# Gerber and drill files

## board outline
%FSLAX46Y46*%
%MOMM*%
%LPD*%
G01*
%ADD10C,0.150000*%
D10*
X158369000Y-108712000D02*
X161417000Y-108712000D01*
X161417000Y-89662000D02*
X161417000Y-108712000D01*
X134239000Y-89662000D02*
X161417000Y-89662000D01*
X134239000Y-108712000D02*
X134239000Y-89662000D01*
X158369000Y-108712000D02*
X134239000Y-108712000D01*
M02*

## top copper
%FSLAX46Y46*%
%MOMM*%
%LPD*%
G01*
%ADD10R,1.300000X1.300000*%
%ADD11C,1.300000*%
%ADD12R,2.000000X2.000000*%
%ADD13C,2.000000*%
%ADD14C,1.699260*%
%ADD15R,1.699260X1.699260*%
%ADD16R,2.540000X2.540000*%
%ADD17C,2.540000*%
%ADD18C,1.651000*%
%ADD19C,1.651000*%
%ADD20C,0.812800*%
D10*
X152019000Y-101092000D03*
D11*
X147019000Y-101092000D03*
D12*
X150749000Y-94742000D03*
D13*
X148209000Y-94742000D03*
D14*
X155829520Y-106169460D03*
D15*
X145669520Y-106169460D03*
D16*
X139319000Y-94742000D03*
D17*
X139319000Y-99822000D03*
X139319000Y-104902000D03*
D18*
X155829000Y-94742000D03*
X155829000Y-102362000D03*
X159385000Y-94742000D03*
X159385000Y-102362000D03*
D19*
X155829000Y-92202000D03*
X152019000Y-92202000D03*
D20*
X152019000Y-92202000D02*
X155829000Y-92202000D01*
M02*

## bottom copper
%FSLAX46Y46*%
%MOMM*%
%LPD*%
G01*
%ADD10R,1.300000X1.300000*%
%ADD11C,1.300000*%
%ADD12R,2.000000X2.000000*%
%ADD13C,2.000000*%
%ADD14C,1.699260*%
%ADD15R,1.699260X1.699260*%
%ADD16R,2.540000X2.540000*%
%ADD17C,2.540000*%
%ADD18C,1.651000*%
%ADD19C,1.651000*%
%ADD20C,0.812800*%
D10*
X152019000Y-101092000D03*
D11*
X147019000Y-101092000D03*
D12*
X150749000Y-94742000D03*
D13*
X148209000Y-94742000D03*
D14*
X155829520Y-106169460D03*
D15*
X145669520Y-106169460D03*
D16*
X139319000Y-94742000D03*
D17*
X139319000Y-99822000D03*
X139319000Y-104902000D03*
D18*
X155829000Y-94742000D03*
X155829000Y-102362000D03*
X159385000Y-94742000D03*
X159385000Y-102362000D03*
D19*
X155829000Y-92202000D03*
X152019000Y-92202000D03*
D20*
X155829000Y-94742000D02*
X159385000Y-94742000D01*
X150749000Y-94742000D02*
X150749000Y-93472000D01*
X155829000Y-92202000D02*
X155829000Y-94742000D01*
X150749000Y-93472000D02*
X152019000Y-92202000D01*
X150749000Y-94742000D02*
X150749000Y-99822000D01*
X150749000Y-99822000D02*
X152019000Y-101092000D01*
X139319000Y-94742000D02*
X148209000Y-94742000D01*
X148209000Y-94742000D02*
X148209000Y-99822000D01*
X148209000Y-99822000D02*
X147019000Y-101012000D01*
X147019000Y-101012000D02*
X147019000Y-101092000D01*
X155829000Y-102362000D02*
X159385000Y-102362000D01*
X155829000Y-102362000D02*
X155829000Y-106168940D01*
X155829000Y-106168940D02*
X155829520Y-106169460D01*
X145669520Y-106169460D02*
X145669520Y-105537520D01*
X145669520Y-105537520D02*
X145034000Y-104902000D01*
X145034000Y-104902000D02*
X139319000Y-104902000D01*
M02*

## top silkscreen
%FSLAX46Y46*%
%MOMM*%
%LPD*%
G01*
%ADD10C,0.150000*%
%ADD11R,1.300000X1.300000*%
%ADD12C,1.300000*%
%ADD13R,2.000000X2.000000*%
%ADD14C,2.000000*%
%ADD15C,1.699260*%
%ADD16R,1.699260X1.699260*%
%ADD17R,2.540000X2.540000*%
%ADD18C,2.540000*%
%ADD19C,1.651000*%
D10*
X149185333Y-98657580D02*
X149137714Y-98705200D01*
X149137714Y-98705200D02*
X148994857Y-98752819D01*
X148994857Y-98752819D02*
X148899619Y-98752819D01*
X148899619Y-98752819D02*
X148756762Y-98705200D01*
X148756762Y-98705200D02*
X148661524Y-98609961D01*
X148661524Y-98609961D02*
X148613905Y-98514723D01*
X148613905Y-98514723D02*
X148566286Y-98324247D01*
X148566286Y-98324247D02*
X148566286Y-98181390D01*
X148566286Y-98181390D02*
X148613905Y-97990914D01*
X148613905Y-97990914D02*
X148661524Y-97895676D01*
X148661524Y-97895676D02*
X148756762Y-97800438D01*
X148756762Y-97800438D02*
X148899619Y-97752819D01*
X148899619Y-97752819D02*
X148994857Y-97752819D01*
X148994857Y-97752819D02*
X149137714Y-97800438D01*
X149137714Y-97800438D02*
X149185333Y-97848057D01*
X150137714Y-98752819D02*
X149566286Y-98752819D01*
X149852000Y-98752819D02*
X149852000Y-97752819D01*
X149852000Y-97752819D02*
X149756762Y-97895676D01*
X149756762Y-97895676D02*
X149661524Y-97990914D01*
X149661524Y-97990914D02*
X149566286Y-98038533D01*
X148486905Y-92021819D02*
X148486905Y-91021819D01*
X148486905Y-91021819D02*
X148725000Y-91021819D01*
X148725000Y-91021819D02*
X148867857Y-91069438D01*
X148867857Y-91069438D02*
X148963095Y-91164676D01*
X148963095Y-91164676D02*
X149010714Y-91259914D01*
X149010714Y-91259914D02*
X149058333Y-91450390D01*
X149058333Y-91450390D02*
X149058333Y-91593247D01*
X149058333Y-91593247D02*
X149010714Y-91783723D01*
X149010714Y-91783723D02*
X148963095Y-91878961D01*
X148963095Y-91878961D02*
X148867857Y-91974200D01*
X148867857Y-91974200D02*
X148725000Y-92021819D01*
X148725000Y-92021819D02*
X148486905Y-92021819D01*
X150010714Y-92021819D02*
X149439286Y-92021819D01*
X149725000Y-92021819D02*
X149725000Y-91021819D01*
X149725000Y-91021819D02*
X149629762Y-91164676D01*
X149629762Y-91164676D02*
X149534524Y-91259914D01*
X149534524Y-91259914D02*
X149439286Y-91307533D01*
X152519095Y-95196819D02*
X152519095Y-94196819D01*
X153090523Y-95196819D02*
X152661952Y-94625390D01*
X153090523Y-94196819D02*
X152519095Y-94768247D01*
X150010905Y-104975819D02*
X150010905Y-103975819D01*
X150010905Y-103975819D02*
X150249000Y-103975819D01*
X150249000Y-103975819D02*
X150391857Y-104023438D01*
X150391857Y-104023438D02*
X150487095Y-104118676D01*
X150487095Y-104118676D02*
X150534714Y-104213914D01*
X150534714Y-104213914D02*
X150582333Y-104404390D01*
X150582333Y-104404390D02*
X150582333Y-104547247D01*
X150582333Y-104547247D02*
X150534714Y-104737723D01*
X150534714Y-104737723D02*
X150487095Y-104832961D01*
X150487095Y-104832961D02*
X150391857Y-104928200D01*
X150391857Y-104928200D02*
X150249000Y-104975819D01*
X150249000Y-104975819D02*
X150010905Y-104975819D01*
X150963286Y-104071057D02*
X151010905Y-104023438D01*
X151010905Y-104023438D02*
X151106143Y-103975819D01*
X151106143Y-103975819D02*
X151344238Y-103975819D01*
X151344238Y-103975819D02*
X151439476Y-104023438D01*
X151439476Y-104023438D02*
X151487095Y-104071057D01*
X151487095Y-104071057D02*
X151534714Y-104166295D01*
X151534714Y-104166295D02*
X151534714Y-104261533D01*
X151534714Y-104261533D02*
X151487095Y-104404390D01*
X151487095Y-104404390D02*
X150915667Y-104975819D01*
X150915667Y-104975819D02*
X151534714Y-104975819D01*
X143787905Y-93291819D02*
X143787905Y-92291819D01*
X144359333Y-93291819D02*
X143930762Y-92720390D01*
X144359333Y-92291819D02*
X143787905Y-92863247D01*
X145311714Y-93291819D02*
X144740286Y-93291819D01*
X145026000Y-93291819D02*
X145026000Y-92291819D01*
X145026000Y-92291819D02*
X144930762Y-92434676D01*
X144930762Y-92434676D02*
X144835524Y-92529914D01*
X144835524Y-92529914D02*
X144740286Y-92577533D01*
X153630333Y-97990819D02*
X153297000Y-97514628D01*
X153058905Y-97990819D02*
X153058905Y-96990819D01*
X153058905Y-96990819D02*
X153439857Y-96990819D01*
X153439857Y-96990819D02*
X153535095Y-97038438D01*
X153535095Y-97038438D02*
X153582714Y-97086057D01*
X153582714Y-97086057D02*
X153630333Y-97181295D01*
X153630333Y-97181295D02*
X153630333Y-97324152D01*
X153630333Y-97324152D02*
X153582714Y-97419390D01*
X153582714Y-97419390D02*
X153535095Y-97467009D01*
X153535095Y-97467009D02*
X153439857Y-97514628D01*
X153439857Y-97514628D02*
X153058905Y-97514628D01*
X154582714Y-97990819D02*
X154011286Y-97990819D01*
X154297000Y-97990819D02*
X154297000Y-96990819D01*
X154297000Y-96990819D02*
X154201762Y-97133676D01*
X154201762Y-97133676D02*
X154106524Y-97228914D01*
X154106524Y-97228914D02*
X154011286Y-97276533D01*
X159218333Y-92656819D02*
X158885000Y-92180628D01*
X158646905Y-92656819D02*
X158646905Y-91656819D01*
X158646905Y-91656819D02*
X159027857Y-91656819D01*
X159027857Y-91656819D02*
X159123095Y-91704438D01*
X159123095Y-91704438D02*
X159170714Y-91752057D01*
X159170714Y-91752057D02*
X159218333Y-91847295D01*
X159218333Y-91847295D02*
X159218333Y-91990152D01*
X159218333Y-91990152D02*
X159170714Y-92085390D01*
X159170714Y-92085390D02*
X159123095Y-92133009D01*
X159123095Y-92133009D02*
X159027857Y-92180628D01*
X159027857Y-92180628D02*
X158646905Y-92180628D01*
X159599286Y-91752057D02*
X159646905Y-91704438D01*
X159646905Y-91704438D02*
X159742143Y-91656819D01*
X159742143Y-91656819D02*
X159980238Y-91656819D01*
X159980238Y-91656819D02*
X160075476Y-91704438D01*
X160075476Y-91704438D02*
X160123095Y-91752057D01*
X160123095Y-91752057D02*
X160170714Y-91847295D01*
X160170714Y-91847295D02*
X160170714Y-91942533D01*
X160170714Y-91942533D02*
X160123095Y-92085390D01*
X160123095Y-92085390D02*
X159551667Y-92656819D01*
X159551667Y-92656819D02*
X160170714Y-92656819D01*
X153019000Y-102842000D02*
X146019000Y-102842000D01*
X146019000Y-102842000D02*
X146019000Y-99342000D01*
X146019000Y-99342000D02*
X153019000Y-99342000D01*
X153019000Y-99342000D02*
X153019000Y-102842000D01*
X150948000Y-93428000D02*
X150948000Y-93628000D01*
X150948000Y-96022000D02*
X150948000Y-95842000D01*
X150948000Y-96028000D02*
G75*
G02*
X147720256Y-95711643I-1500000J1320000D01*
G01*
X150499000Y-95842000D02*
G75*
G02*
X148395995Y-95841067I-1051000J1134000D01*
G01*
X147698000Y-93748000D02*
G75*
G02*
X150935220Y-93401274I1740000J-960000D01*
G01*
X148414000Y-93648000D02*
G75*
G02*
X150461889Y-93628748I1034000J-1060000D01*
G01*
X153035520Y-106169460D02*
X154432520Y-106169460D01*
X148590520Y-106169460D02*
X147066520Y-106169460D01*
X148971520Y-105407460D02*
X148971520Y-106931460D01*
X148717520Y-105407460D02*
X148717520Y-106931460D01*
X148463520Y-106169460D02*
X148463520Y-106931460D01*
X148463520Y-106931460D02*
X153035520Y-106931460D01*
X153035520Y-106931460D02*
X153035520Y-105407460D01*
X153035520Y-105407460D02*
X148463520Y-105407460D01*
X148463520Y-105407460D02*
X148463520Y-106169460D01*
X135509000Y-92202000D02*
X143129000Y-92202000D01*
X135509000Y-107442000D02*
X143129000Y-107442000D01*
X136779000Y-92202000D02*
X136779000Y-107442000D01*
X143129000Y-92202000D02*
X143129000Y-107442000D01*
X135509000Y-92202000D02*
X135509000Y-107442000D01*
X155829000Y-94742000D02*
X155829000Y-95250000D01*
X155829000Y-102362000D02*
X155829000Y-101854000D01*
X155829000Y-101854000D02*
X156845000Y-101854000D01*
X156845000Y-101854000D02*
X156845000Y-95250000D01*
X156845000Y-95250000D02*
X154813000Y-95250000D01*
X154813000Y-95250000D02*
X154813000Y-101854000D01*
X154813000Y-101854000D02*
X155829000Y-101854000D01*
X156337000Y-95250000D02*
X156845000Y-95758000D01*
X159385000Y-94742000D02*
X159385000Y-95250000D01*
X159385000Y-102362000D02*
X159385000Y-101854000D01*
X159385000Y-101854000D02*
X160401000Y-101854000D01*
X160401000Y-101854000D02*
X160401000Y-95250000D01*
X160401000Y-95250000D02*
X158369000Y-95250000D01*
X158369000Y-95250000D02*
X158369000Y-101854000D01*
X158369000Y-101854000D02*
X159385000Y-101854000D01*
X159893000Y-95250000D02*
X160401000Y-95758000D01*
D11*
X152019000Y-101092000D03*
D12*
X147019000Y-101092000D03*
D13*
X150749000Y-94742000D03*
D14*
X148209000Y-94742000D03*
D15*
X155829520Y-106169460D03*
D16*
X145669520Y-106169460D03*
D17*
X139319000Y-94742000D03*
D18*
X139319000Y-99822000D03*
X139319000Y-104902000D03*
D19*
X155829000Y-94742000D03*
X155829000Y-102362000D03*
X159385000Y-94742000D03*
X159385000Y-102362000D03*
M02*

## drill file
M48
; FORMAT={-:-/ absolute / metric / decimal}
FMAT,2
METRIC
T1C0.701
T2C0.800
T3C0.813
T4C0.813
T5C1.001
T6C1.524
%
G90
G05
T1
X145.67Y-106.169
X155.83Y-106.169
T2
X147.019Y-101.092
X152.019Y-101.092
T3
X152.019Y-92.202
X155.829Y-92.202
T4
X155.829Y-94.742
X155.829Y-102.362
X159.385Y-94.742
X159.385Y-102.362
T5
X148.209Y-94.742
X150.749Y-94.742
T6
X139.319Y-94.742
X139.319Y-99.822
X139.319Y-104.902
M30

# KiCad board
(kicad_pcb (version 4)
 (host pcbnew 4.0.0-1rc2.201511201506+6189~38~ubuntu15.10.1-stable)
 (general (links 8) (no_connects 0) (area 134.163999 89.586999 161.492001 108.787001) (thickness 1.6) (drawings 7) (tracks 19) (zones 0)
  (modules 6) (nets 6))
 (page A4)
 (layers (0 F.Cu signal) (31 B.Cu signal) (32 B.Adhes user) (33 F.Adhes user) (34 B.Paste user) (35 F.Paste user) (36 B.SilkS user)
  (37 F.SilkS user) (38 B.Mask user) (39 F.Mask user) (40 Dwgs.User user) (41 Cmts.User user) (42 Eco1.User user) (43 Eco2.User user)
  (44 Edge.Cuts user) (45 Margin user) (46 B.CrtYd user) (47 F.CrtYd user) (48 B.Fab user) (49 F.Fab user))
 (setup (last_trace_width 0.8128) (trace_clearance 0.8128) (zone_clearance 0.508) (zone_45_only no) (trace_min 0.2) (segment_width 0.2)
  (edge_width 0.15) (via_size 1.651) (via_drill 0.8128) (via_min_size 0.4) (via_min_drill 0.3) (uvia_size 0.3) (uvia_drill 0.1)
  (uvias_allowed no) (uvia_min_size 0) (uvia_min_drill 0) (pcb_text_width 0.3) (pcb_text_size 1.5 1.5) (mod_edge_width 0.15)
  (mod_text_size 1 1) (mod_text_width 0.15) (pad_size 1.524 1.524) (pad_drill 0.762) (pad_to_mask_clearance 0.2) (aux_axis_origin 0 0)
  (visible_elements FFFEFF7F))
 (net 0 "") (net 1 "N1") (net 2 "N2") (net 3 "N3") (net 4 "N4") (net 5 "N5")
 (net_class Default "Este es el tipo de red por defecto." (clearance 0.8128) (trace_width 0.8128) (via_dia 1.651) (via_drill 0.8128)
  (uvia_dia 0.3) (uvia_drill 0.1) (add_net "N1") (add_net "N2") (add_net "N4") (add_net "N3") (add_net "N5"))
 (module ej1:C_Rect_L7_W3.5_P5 (layer F.Cu) (at 152.019 101.092 180)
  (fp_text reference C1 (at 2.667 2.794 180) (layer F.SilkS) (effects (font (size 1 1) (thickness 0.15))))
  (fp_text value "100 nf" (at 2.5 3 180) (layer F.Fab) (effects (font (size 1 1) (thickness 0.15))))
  (fp_line (start -1 -1.75) (end 6 -1.75) (layer F.SilkS) (width 0.15))
  (fp_line (start 6 -1.75) (end 6 1.75) (layer F.SilkS) (width 0.15))
  (fp_line (start 6 1.75) (end -1 1.75) (layer F.SilkS) (width 0.15))
  (fp_line (start -1 1.75) (end -1 -1.75) (layer F.SilkS) (width 0.15))
  (pad 1 thru_hole rect (at 0 0 180) (size 1.3 1.3) (drill 0.8) (layers *.Cu *.Mask F.SilkS) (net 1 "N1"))
  (pad 2 thru_hole circle (at 5 0 180) (size 1.3 1.3) (drill 0.8) (layers *.Cu *.Mask F.SilkS) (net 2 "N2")))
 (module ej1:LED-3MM (layer F.Cu) (at 150.749 94.742 180)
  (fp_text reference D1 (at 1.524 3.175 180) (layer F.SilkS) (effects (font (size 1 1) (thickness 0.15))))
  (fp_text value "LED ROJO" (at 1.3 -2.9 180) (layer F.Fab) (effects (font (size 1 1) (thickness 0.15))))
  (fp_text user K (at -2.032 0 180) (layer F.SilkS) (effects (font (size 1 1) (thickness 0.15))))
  (fp_line (start -0.199 1.314) (end -0.199 1.114) (layer F.SilkS) (width 0.15))
  (fp_line (start -0.199 -1.28) (end -0.199 -1.1) (layer F.SilkS) (width 0.15))
  (fp_arc (start 1.301 0.034) (end -0.199 -1.286) (angle 108.5) (layer F.SilkS) (width 0.15))
  (fp_arc (start 1.301 0.034) (end 0.25 -1.1) (angle 85.7) (layer F.SilkS) (width 0.15))
  (fp_arc (start 1.311 0.034) (end 3.051 0.994) (angle 110) (layer F.SilkS) (width 0.15))
  (fp_arc (start 1.301 0.034) (end 2.335 1.094) (angle 87.5) (layer F.SilkS) (width 0.15))
  (pad 1 thru_hole rect (at 0 0 270) (size 2 2) (drill 1.00076) (layers *.Cu *.Mask F.SilkS) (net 1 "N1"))
  (pad 2 thru_hole circle (at 2.54 0 180) (size 2 2) (drill 1.00076) (layers *.Cu *.Mask F.SilkS) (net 2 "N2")))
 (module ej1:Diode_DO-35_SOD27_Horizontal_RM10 (layer F.Cu) (at 145.669 106.172)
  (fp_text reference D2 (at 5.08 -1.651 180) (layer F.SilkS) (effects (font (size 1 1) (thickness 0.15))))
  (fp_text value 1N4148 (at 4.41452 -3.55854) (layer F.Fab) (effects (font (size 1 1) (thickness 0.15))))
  (fp_line (start 7.36652 -0.00254) (end 8.76352 -0.00254) (layer F.SilkS) (width 0.15))
  (fp_line (start 2.92152 -0.00254) (end 1.39752 -0.00254) (layer F.SilkS) (width 0.15))
  (fp_line (start 3.30252 -0.76454) (end 3.30252 0.75946) (layer F.SilkS) (width 0.15))
  (fp_line (start 3.04852 -0.76454) (end 3.04852 0.75946) (layer F.SilkS) (width 0.15))
  (fp_line (start 2.79452 -0.00254) (end 2.79452 0.75946) (layer F.SilkS) (width 0.15))
  (fp_line (start 2.79452 0.75946) (end 7.36652 0.75946) (layer F.SilkS) (width 0.15))
  (fp_line (start 7.36652 0.75946) (end 7.36652 -0.76454) (layer F.SilkS) (width 0.15))
  (fp_line (start 7.36652 -0.76454) (end 2.79452 -0.76454) (layer F.SilkS) (width 0.15))
  (fp_line (start 2.79452 -0.76454) (end 2.79452 -0.00254) (layer F.SilkS) (width 0.15))
  (pad 2 thru_hole circle (at 10.16052 -0.00254 180) (size 1.69926 1.69926) (drill 0.70104) (layers *.Cu *.Mask F.SilkS) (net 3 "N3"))
  (pad 1 thru_hole rect (at 0.00052 -0.00254 180) (size 1.69926 1.69926) (drill 0.70104) (layers *.Cu *.Mask F.SilkS) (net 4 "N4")))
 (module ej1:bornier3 (layer F.Cu) (at 139.319 99.822 270)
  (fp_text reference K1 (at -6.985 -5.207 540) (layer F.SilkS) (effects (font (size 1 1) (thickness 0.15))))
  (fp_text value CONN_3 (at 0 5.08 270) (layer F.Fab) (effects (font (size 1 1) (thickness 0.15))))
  (fp_line (start -7.62 3.81) (end -7.62 -3.81) (layer F.SilkS) (width 0.15))
  (fp_line (start 7.62 3.81) (end 7.62 -3.81) (layer F.SilkS) (width 0.15))
  (fp_line (start -7.62 2.54) (end 7.62 2.54) (layer F.SilkS) (width 0.15))
  (fp_line (start -7.62 -3.81) (end 7.62 -3.81) (layer F.SilkS) (width 0.15))
  (fp_line (start -7.62 3.81) (end 7.62 3.81) (layer F.SilkS) (width 0.15))
  (pad 1 thru_hole rect (at -5.08 0 270) (size 2.54 2.54) (drill 1.524) (layers *.Cu *.Mask F.SilkS) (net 2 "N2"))
  (pad 2 thru_hole circle (at 0 0 270) (size 2.54 2.54) (drill 1.524) (layers *.Cu *.Mask F.SilkS) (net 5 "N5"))
  (pad 3 thru_hole circle (at 5.08 0 270) (size 2.54 2.54) (drill 1.524) (layers *.Cu *.Mask F.SilkS) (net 4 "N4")))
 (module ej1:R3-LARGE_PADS (layer F.Cu) (at 155.829 98.552 270)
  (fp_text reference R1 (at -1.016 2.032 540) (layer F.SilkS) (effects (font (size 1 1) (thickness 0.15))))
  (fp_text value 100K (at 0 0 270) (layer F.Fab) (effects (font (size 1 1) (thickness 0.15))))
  (fp_line (start -3.81 0) (end -3.302 0) (layer F.SilkS) (width 0.15))
  (fp_line (start 3.81 0) (end 3.302 0) (layer F.SilkS) (width 0.15))
  (fp_line (start 3.302 0) (end 3.302 -1.016) (layer F.SilkS) (width 0.15))
  (fp_line (start 3.302 -1.016) (end -3.302 -1.016) (layer F.SilkS) (width 0.15))
  (fp_line (start -3.302 -1.016) (end -3.302 1.016) (layer F.SilkS) (width 0.15))
  (fp_line (start -3.302 1.016) (end 3.302 1.016) (layer F.SilkS) (width 0.15))
  (fp_line (start 3.302 1.016) (end 3.302 0) (layer F.SilkS) (width 0.15))
  (fp_line (start -3.302 -0.508) (end -2.794 -1.016) (layer F.SilkS) (width 0.15))
  (pad 1 thru_hole circle (at -3.81 0 270) (size 1.651 1.651) (drill 0.8128) (layers *.Cu *.Mask F.SilkS) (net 1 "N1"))
  (pad 2 thru_hole circle (at 3.81 0 270) (size 1.651 1.651) (drill 0.8128) (layers *.Cu *.Mask F.SilkS) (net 3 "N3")))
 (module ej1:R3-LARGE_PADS (layer F.Cu) (at 159.385 98.552 270)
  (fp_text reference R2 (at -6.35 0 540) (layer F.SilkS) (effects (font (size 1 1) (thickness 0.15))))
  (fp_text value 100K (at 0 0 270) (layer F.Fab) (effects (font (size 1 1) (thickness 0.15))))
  (fp_line (start -3.81 0) (end -3.302 0) (layer F.SilkS) (width 0.15))
  (fp_line (start 3.81 0) (end 3.302 0) (layer F.SilkS) (width 0.15))
  (fp_line (start 3.302 0) (end 3.302 -1.016) (layer F.SilkS) (width 0.15))
  (fp_line (start 3.302 -1.016) (end -3.302 -1.016) (layer F.SilkS) (width 0.15))
  (fp_line (start -3.302 -1.016) (end -3.302 1.016) (layer F.SilkS) (width 0.15))
  (fp_line (start -3.302 1.016) (end 3.302 1.016) (layer F.SilkS) (width 0.15))
  (fp_line (start 3.302 1.016) (end 3.302 0) (layer F.SilkS) (width 0.15))
  (fp_line (start -3.302 -0.508) (end -2.794 -1.016) (layer F.SilkS) (width 0.15))
  (pad 1 thru_hole circle (at -3.81 0 270) (size 1.651 1.651) (drill 0.8128) (layers *.Cu *.Mask F.SilkS) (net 1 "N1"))
  (pad 2 thru_hole circle (at 3.81 0 270) (size 1.651 1.651) (drill 0.8128) (layers *.Cu *.Mask F.SilkS) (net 3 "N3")))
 (gr_line (start 158.369 108.712) (end 161.417 108.712) (angle 90) (layer Edge.Cuts) (width 0.15))
 (gr_line (start 161.417 89.662) (end 161.417 108.712) (angle 90) (layer Edge.Cuts) (width 0.15))
 (gr_line (start 134.239 89.662) (end 161.417 89.662) (angle 90) (layer Edge.Cuts) (width 0.15))
 (gr_line (start 134.239 108.712) (end 134.239 89.662) (angle 90) (layer Edge.Cuts) (width 0.15))
 (gr_line (start 158.369 108.712) (end 134.239 108.712) (angle 90) (layer Edge.Cuts) (width 0.15))
 (segment (start 155.829 94.742) (end 159.385 94.742) (width 0.8128) (layer B.Cu) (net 1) (status C00000))
 (segment (start 150.749 94.742) (end 150.749 93.472) (width 0.8128) (layer B.Cu) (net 1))
 (segment (start 155.829 92.202) (end 155.829 94.742) (width 0.8128) (layer B.Cu) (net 1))
 (segment (start 152.019 92.202) (end 155.829 92.202) (width 0.8128) (layer F.Cu) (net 1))
 (segment (start 150.749 93.472) (end 152.019 92.202) (width 0.8128) (layer B.Cu) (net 1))
 (segment (start 150.749 94.742) (end 150.749 99.822) (width 0.8128) (layer B.Cu) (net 1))
 (segment (start 150.749 99.822) (end 152.019 101.092) (width 0.8128) (layer B.Cu) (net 1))
 (segment (start 139.319 94.742) (end 148.209 94.742) (width 0.8128) (layer B.Cu) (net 2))
 (segment (start 148.209 94.742) (end 148.209 99.822) (width 0.8128) (layer B.Cu) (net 2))
 (segment (start 148.209 99.822) (end 147.019 101.012) (width 0.8128) (layer B.Cu) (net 2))
 (segment (start 147.019 101.012) (end 147.019 101.092) (width 0.8128) (layer B.Cu) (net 2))
 (segment (start 155.829 102.362) (end 159.385 102.362) (width 0.8128) (layer B.Cu) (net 3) (status C00000))
 (segment (start 155.829 102.362) (end 155.829 106.16894) (width 0.8128) (layer B.Cu) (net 3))
 (segment (start 155.829 106.16894) (end 155.82952 106.16946) (width 0.8128) (layer B.Cu) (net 3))
 (segment (start 145.66952 106.16946) (end 145.66952 105.53752) (width 0.8128) (layer B.Cu) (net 4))
 (segment (start 145.66952 105.53752) (end 145.034 104.902) (width 0.8128) (layer B.Cu) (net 4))
 (segment (start 145.034 104.902) (end 139.319 104.902) (width 0.8128) (layer B.Cu) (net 4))
 (via (at 155.829 92.202) (size 1.651) (drill 0.8128) (layers F.Cu B.Cu) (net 1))
 (via (at 152.019 92.202) (size 1.651) (drill 0.8128) (layers F.Cu B.Cu) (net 1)))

